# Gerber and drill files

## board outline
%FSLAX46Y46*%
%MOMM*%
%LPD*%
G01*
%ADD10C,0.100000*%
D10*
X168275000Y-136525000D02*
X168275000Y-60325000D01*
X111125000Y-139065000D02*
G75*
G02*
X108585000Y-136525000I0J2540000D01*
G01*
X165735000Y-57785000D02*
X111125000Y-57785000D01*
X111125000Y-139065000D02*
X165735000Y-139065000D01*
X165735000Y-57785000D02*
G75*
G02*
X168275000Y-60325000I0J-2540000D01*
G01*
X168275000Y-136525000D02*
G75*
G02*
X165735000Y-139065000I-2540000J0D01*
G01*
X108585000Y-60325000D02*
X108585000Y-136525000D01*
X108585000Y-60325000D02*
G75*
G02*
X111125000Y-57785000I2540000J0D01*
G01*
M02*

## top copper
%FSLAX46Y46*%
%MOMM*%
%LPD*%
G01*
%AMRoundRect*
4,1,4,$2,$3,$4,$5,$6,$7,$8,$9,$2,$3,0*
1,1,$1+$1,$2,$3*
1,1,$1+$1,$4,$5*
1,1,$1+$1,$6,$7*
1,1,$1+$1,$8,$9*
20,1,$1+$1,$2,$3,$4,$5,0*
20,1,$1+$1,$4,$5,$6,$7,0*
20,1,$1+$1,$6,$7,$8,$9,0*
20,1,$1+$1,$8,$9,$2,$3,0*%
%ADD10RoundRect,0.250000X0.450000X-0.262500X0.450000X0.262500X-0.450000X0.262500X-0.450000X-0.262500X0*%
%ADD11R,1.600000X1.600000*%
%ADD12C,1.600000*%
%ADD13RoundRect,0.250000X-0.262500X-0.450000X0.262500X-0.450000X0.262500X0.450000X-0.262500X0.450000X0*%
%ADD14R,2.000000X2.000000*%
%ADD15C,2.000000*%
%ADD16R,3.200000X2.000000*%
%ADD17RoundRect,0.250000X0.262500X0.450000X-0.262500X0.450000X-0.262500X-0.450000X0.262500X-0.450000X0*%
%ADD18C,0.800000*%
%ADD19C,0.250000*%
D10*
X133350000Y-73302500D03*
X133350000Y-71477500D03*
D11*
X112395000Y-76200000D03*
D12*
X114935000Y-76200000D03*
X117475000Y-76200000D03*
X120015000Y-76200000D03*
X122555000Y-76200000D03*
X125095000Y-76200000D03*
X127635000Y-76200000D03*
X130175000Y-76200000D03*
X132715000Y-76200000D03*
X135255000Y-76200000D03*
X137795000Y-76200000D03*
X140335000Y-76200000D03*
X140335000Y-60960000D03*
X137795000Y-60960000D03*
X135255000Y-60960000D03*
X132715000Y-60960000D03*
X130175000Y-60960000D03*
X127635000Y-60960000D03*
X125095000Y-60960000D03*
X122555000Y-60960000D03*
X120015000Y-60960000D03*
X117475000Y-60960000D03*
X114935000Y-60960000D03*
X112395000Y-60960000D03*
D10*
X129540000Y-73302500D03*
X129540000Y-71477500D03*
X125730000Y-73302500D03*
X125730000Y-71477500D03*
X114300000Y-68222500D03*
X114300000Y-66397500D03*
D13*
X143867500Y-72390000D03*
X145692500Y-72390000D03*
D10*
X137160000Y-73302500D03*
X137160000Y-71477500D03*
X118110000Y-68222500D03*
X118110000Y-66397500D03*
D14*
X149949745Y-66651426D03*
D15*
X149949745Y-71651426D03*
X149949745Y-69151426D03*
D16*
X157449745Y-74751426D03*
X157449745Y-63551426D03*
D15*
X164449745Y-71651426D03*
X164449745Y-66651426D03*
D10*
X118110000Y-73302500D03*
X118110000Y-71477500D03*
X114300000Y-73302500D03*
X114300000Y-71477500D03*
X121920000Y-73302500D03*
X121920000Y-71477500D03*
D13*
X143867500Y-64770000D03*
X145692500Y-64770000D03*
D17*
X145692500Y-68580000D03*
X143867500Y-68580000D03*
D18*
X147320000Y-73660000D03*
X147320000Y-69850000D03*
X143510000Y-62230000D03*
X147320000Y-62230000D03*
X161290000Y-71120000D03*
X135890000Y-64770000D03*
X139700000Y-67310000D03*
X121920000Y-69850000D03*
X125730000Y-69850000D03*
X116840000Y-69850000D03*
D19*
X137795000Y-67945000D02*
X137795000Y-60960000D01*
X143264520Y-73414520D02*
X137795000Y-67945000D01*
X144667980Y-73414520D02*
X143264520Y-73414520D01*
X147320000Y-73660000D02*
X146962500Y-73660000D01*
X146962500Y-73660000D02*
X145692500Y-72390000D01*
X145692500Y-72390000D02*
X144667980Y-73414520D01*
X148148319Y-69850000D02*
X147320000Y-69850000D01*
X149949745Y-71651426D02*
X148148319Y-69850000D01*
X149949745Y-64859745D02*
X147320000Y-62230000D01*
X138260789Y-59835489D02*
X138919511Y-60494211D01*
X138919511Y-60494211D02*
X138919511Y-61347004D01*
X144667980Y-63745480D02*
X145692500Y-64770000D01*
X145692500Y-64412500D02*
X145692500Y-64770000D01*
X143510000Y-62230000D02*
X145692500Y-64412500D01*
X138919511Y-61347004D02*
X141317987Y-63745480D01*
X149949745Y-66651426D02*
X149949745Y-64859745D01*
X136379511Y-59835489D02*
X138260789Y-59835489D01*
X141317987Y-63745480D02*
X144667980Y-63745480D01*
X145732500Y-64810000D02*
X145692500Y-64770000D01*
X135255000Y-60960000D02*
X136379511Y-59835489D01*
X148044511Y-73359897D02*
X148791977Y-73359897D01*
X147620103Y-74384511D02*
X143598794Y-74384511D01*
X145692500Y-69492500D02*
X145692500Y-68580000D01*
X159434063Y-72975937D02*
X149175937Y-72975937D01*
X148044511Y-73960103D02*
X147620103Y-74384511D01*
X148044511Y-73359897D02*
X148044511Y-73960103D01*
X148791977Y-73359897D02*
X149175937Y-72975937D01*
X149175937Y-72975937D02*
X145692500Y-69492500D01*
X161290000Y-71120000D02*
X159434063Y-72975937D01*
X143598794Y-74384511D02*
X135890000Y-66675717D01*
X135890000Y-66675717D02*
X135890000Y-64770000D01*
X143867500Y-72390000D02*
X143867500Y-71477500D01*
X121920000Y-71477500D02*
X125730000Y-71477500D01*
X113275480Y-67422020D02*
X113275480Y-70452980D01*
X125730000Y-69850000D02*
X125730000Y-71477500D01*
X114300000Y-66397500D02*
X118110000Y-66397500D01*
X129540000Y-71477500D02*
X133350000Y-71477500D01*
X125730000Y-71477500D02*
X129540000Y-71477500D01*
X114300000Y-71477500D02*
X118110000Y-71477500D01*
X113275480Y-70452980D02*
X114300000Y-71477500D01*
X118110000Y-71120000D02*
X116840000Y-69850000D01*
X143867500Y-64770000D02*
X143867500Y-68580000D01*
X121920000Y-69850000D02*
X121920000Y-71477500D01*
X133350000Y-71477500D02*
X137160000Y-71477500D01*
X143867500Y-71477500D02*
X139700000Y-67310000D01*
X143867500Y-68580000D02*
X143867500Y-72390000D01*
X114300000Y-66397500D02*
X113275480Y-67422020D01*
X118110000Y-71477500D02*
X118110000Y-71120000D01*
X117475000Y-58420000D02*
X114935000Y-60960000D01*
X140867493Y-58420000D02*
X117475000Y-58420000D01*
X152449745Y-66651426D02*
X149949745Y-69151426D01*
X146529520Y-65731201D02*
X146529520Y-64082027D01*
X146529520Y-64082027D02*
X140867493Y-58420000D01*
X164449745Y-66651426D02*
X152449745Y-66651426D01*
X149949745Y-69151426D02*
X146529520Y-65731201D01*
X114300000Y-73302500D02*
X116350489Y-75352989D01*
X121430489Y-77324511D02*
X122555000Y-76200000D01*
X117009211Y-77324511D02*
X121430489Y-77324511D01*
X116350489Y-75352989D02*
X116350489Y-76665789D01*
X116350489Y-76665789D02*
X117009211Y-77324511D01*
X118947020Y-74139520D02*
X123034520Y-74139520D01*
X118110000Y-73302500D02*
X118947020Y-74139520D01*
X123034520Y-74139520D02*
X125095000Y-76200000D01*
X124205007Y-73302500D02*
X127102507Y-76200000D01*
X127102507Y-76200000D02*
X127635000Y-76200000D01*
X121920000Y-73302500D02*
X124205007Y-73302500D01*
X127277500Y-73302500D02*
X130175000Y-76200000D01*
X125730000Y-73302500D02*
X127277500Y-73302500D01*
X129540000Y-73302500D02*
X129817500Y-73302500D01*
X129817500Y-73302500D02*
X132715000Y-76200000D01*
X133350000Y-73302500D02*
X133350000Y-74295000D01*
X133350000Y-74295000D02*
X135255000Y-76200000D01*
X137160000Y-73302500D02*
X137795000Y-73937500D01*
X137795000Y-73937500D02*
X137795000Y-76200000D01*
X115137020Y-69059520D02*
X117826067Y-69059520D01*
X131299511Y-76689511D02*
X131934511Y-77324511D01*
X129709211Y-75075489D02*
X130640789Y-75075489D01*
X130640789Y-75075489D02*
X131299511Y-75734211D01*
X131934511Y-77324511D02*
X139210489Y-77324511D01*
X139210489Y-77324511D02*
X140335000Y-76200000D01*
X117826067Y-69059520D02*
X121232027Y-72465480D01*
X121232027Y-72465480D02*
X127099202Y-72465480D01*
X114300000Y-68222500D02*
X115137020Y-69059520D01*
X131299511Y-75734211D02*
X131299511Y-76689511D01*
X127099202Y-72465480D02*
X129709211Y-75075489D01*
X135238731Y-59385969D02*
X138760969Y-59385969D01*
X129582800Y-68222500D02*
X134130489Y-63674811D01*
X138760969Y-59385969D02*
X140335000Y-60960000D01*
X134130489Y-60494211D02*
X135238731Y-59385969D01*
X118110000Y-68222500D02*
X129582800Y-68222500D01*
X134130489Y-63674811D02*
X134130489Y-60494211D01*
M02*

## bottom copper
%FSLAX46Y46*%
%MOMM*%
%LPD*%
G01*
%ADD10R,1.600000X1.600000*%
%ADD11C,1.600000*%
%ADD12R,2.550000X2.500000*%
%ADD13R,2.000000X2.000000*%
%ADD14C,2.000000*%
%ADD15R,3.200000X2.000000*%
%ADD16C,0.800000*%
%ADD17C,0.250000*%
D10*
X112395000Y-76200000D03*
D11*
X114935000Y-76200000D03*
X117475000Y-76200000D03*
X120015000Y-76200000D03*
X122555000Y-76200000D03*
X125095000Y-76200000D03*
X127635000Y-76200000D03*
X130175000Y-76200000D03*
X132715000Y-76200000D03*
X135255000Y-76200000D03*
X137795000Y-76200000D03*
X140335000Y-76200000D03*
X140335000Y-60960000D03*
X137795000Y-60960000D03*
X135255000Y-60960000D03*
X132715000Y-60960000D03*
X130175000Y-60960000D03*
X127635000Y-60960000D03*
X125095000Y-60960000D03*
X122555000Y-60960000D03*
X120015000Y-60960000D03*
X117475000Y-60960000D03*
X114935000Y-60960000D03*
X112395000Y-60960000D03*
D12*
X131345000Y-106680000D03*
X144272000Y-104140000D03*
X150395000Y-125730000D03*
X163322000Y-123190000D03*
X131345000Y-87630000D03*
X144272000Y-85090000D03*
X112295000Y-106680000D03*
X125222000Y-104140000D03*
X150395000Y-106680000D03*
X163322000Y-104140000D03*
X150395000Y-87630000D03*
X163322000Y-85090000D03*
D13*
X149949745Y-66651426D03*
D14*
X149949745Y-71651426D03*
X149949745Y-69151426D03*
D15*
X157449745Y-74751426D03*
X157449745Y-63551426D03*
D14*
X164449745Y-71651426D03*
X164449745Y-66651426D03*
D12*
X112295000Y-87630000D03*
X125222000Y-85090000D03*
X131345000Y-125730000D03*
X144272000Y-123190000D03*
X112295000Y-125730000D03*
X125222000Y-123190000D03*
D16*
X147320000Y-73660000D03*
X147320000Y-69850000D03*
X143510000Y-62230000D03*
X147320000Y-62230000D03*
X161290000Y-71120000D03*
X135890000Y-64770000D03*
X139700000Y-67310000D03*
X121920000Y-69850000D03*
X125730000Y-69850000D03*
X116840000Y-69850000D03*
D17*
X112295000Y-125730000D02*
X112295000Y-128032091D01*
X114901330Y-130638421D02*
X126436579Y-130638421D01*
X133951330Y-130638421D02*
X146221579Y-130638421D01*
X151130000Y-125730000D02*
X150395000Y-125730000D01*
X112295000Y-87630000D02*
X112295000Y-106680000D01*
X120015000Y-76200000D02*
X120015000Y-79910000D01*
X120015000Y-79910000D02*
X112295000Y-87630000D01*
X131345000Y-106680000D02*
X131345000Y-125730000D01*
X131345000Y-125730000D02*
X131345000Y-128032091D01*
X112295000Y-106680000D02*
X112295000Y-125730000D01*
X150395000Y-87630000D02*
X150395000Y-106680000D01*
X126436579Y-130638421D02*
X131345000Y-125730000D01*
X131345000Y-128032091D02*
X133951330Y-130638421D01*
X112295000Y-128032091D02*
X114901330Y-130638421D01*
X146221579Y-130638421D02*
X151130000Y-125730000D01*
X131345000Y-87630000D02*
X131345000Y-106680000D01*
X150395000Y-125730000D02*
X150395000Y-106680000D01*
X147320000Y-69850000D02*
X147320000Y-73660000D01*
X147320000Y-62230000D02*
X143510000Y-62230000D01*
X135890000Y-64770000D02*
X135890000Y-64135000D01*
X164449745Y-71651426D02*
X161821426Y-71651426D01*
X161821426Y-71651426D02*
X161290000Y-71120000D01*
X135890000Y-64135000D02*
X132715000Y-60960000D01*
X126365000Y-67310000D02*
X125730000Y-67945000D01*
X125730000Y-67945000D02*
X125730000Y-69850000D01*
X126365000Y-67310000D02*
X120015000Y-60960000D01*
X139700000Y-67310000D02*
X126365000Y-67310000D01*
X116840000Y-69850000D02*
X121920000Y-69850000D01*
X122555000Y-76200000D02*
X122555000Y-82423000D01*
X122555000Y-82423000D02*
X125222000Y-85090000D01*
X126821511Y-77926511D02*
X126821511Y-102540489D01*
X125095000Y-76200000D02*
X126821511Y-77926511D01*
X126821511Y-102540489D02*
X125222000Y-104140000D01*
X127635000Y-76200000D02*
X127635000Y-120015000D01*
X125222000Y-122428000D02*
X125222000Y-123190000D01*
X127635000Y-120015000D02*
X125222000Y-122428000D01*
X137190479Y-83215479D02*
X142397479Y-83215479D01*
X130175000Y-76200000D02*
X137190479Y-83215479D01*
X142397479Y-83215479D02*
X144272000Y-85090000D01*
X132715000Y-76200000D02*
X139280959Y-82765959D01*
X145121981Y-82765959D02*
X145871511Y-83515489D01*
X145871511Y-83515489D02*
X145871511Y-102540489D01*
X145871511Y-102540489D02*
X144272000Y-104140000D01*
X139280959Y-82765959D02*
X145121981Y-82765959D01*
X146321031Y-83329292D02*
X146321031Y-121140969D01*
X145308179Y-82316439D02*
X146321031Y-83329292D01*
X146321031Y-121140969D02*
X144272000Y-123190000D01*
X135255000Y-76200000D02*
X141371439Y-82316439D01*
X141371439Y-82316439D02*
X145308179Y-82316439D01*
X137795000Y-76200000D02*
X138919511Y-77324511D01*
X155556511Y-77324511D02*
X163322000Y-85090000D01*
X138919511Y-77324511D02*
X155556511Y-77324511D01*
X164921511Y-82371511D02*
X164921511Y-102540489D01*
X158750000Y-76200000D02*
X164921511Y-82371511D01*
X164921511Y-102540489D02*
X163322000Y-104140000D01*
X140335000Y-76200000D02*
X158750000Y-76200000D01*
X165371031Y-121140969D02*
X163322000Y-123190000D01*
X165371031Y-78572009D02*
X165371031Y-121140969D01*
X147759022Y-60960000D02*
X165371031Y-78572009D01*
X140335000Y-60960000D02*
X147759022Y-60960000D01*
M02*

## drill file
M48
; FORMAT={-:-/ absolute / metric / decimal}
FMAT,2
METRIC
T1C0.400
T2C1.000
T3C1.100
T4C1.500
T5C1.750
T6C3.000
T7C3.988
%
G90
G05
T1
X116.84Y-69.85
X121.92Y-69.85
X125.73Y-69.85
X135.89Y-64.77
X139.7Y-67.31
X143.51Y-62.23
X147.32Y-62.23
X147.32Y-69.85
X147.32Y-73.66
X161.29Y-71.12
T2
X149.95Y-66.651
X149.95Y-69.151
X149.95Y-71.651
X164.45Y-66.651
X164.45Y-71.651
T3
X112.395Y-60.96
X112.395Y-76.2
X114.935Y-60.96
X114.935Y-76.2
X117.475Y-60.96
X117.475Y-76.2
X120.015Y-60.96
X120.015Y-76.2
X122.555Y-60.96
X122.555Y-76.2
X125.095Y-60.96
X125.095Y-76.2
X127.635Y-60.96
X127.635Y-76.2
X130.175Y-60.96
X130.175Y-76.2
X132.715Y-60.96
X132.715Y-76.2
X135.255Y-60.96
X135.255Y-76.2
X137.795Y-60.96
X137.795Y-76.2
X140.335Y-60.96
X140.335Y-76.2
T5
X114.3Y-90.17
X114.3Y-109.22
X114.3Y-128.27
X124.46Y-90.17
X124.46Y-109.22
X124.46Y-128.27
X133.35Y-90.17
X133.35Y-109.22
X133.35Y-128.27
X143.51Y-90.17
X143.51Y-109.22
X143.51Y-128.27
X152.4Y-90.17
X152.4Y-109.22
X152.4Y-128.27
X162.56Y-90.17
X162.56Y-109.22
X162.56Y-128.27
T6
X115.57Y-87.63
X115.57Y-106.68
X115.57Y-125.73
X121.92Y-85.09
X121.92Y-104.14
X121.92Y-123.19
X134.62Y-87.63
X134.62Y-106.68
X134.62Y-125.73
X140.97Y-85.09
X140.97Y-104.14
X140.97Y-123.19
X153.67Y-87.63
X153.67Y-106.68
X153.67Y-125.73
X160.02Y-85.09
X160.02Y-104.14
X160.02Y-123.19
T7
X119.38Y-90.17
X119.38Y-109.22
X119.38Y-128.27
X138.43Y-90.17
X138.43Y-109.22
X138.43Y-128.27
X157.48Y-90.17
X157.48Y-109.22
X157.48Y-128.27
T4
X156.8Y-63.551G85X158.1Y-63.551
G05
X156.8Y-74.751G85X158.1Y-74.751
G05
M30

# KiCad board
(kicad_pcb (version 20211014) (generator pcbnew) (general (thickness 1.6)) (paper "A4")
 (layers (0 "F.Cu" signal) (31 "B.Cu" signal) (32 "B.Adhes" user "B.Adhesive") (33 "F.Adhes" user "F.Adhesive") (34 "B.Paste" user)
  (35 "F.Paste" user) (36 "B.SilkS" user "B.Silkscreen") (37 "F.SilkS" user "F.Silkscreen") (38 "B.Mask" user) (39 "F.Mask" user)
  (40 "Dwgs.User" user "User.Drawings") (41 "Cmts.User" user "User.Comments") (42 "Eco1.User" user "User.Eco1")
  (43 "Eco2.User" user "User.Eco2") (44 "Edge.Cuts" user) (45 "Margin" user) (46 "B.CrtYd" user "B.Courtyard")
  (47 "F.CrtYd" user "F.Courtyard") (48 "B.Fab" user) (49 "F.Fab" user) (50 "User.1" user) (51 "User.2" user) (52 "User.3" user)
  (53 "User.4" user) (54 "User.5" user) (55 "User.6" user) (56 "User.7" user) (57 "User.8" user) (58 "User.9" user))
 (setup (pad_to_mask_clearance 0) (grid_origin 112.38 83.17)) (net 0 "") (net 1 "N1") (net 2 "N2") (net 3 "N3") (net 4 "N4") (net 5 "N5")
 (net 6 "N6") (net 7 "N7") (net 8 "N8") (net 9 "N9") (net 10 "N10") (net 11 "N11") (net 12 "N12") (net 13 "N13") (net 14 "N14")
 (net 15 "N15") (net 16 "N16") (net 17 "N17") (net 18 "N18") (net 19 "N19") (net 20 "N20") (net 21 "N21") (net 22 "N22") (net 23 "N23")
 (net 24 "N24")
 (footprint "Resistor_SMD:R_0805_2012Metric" (layer "F.Cu") (at 133.35 72.39 90)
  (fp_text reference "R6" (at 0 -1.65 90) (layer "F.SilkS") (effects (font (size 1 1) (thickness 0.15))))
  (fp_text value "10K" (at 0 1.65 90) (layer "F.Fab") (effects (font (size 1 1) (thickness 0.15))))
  (pad "1" smd roundrect locked (at -0.9125 0 90) (size 1.025 1.4) (layers "F.Cu" "F.Paste" "F.Mask") (roundrect_rratio 0.243902439)
   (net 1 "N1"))
  (pad "2" smd roundrect locked (at 0.9125 0 90) (size 1.025 1.4) (layers "F.Cu" "F.Paste" "F.Mask") (roundrect_rratio 0.243902439)
   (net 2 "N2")))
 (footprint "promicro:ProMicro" (layer "F.Cu") (at 126.365 68.58)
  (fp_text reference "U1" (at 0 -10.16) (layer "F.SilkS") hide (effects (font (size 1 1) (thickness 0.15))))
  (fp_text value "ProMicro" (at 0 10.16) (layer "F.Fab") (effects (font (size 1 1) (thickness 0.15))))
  (pad "1" thru_hole rect locked (at -13.97 7.62) (size 1.6 1.6) (drill 1.1) (layers *.Cu *.Mask "F.SilkS") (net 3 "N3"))
  (pad "2" thru_hole circle locked (at -11.43 7.62) (size 1.6 1.6) (drill 1.1) (layers *.Cu *.Mask "F.SilkS") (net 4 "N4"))
  (pad "3" thru_hole circle locked (at -8.89 7.62) (size 1.6 1.6) (drill 1.1) (layers *.Cu *.Mask "F.SilkS") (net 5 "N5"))
  (pad "4" thru_hole circle locked (at -6.35 7.62) (size 1.6 1.6) (drill 1.1) (layers *.Cu *.Mask "F.SilkS") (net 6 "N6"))
  (pad "5" thru_hole circle locked (at -3.81 7.62) (size 1.6 1.6) (drill 1.1) (layers *.Cu *.Mask "F.SilkS") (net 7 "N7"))
  (pad "6" thru_hole circle locked (at -1.27 7.62) (size 1.6 1.6) (drill 1.1) (layers *.Cu *.Mask "F.SilkS") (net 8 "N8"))
  (pad "7" thru_hole circle locked (at 1.27 7.62) (size 1.6 1.6) (drill 1.1) (layers *.Cu *.Mask "F.SilkS") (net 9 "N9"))
  (pad "8" thru_hole circle locked (at 3.81 7.62) (size 1.6 1.6) (drill 1.1) (layers *.Cu *.Mask "F.SilkS") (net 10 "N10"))
  (pad "9" thru_hole circle locked (at 6.35 7.62) (size 1.6 1.6) (drill 1.1) (layers *.Cu *.Mask "F.SilkS") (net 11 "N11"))
  (pad "10" thru_hole circle locked (at 8.89 7.62) (size 1.6 1.6) (drill 1.1) (layers *.Cu *.Mask "F.SilkS") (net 1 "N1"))
  (pad "11" thru_hole circle locked (at 11.43 7.62) (size 1.6 1.6) (drill 1.1) (layers *.Cu *.Mask "F.SilkS") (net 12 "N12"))
  (pad "12" thru_hole circle locked (at 13.97 7.62) (size 1.6 1.6) (drill 1.1) (layers *.Cu *.Mask "F.SilkS") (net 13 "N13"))
  (pad "13" thru_hole circle locked (at 13.97 -7.62) (size 1.6 1.6) (drill 1.1) (layers *.Cu *.Mask "F.SilkS") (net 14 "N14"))
  (pad "14" thru_hole circle locked (at 11.43 -7.62) (size 1.6 1.6) (drill 1.1) (layers *.Cu *.Mask "F.SilkS") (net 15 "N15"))
  (pad "15" thru_hole circle locked (at 8.89 -7.62) (size 1.6 1.6) (drill 1.1) (layers *.Cu *.Mask "F.SilkS") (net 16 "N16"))
  (pad "16" thru_hole circle locked (at 6.35 -7.62) (size 1.6 1.6) (drill 1.1) (layers *.Cu *.Mask "F.SilkS") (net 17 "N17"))
  (pad "17" thru_hole circle locked (at 3.81 -7.62) (size 1.6 1.6) (drill 1.1) (layers *.Cu *.Mask "F.SilkS") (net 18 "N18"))
  (pad "18" thru_hole circle locked (at 1.27 -7.62) (size 1.6 1.6) (drill 1.1) (layers *.Cu *.Mask "F.SilkS") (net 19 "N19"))
  (pad "19" thru_hole circle locked (at -1.27 -7.62) (size 1.6 1.6) (drill 1.1) (layers *.Cu *.Mask "F.SilkS") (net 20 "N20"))
  (pad "20" thru_hole circle locked (at -3.81 -7.62) (size 1.6 1.6) (drill 1.1) (layers *.Cu *.Mask "F.SilkS") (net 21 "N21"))
  (pad "21" thru_hole circle locked (at -6.35 -7.62) (size 1.6 1.6) (drill 1.1) (layers *.Cu *.Mask "F.SilkS") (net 2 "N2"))
  (pad "22" thru_hole circle locked (at -8.89 -7.62) (size 1.6 1.6) (drill 1.1) (layers *.Cu *.Mask "F.SilkS") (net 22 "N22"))
  (pad "23" thru_hole circle locked (at -11.43 -7.62) (size 1.6 1.6) (drill 1.1) (layers *.Cu *.Mask "F.SilkS") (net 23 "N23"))
  (pad "24" thru_hole circle locked (at -13.97 -7.62) (size 1.6 1.6) (drill 1.1) (layers *.Cu *.Mask "F.SilkS") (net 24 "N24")))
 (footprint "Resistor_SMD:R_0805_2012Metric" (layer "F.Cu") (at 129.54 72.39 90)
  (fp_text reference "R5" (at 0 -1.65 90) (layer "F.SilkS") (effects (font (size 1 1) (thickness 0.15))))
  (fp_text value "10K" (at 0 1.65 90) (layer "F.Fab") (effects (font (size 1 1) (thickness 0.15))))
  (pad "1" smd roundrect locked (at -0.9125 0 90) (size 1.025 1.4) (layers "F.Cu" "F.Paste" "F.Mask") (roundrect_rratio 0.243902439)
   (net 11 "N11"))
  (pad "2" smd roundrect locked (at 0.9125 0 90) (size 1.025 1.4) (layers "F.Cu" "F.Paste" "F.Mask") (roundrect_rratio 0.243902439)
   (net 2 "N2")))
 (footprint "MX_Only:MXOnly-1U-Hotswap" (layer "F.Cu") (at 138.43 109.22)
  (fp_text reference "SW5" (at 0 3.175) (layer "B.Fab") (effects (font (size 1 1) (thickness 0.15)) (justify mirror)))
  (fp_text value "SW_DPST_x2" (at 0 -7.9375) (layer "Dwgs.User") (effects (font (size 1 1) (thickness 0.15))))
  (pad "" np_thru_hole circle locked (at -5.08 0 48.0996) (size 1.75 1.75) (drill 1.75) (layers *.Cu *.Mask))
  (pad "" np_thru_hole circle locked (at 0 0) (size 3.9878 3.9878) (drill 3.9878) (layers *.Cu *.Mask))
  (pad "" np_thru_hole circle locked (at -3.81 -2.54) (size 3 3) (drill 3) (layers *.Cu *.Mask))
  (pad "" np_thru_hole circle locked (at 2.54 -5.08) (size 3 3) (drill 3) (layers *.Cu *.Mask))
  (pad "" np_thru_hole circle locked (at 5.08 0 48.0996) (size 1.75 1.75) (drill 1.75) (layers *.Cu *.Mask))
  (pad "1" smd rect locked (at -7.085 -2.54) (size 2.55 2.5) (layers "B.Cu" "B.Paste" "B.Mask") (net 6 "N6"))
  (pad "2" smd rect locked (at 5.842 -5.08) (size 2.55 2.5) (layers "B.Cu" "B.Paste" "B.Mask") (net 11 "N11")))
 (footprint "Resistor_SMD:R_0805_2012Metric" (layer "F.Cu") (at 125.73 72.39 90)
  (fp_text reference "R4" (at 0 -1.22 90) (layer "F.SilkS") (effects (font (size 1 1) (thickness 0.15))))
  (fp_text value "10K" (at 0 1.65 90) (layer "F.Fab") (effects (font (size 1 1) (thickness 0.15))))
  (pad "1" smd roundrect locked (at -0.9125 0 90) (size 1.025 1.4) (layers "F.Cu" "F.Paste" "F.Mask") (roundrect_rratio 0.243902439)
   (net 10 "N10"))
  (pad "2" smd roundrect locked (at 0.9125 0 90) (size 1.025 1.4) (layers "F.Cu" "F.Paste" "F.Mask") (roundrect_rratio 0.243902439)
   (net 2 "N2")))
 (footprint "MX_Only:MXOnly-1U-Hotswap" (layer "F.Cu") (at 157.48 128.27)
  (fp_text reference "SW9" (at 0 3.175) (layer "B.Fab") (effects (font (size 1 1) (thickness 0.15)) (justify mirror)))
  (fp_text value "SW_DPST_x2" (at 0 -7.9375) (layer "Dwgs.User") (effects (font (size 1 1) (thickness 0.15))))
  (pad "" np_thru_hole circle locked (at -5.08 0 48.0996) (size 1.75 1.75) (drill 1.75) (layers *.Cu *.Mask))
  (pad "" np_thru_hole circle locked (at 0 0) (size 3.9878 3.9878) (drill 3.9878) (layers *.Cu *.Mask))
  (pad "" np_thru_hole circle locked (at -3.81 -2.54) (size 3 3) (drill 3) (layers *.Cu *.Mask))
  (pad "" np_thru_hole circle locked (at 5.08 0 48.0996) (size 1.75 1.75) (drill 1.75) (layers *.Cu *.Mask))
  (pad "" np_thru_hole circle locked (at 2.54 -5.08) (size 3 3) (drill 3) (layers *.Cu *.Mask))
  (pad "1" smd rect locked (at -7.085 -2.54) (size 2.55 2.5) (layers "B.Cu" "B.Paste" "B.Mask") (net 6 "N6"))
  (pad "2" smd rect locked (at 5.842 -5.08) (size 2.55 2.5) (layers "B.Cu" "B.Paste" "B.Mask") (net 14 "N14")))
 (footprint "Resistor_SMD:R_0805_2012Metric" (layer "F.Cu") (at 114.3 67.31 90)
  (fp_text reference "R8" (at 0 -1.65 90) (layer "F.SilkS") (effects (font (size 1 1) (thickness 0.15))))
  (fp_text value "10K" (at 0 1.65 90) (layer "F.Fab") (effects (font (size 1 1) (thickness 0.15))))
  (pad "1" smd roundrect locked (at -0.9125 0 90) (size 1.025 1.4) (layers "F.Cu" "F.Paste" "F.Mask") (roundrect_rratio 0.243902439)
   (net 13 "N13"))
  (pad "2" smd roundrect locked (at 0.9125 0 90) (size 1.025 1.4) (layers "F.Cu" "F.Paste" "F.Mask") (roundrect_rratio 0.243902439)
   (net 2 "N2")))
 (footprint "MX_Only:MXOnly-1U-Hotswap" (layer "F.Cu") (at 138.43 90.17)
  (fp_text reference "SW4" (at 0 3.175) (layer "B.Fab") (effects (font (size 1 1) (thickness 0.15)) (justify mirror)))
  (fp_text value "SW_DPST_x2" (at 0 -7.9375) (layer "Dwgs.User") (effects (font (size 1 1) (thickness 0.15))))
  (pad "" np_thru_hole circle locked (at -3.81 -2.54) (size 3 3) (drill 3) (layers *.Cu *.Mask))
  (pad "" np_thru_hole circle locked (at 5.08 0 48.0996) (size 1.75 1.75) (drill 1.75) (layers *.Cu *.Mask))
  (pad "" np_thru_hole circle locked (at 0 0) (size 3.9878 3.9878) (drill 3.9878) (layers *.Cu *.Mask))
  (pad "" np_thru_hole circle locked (at 2.54 -5.08) (size 3 3) (drill 3) (layers *.Cu *.Mask))
  (pad "" np_thru_hole circle locked (at -5.08 0 48.0996) (size 1.75 1.75) (drill 1.75) (layers *.Cu *.Mask))
  (pad "1" smd rect locked (at -7.085 -2.54) (size 2.55 2.5) (layers "B.Cu" "B.Paste" "B.Mask") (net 6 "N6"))
  (pad "2" smd rect locked (at 5.842 -5.08) (size 2.55 2.5) (layers "B.Cu" "B.Paste" "B.Mask") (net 10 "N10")))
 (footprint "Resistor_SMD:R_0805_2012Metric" (layer "F.Cu") (at 144.78 72.39)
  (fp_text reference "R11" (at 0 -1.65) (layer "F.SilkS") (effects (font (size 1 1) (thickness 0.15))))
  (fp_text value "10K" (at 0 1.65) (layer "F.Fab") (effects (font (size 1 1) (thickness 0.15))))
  (pad "1" smd roundrect locked (at -0.9125 0) (size 1.025 1.4) (layers "F.Cu" "F.Paste" "F.Mask") (roundrect_rratio 0.243902439)
   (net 2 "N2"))
  (pad "2" smd roundrect locked (at 0.9125 0) (size 1.025 1.4) (layers "F.Cu" "F.Paste" "F.Mask") (roundrect_rratio 0.243902439)
   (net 15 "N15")))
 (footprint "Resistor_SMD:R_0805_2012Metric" (layer "F.Cu") (at 137.16 72.39 90)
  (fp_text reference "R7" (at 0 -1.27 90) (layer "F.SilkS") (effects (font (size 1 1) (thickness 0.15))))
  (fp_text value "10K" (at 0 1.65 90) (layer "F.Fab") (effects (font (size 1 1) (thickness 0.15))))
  (pad "1" smd roundrect locked (at -0.9125 0 90) (size 1.025 1.4) (layers "F.Cu" "F.Paste" "F.Mask") (roundrect_rratio 0.243902439)
   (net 12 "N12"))
  (pad "2" smd roundrect locked (at 0.9125 0 90) (size 1.025 1.4) (layers "F.Cu" "F.Paste" "F.Mask") (roundrect_rratio 0.243902439)
   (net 2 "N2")))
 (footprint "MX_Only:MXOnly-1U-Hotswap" (layer "F.Cu") (at 119.38 109.22)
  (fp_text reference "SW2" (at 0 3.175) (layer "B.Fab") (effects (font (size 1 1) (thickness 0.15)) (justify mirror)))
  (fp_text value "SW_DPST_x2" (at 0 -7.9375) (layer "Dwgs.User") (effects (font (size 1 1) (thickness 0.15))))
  (pad "" np_thru_hole circle locked (at 2.54 -5.08) (size 3 3) (drill 3) (layers *.Cu *.Mask))
  (pad "" np_thru_hole circle locked (at 5.08 0 48.0996) (size 1.75 1.75) (drill 1.75) (layers *.Cu *.Mask))
  (pad "" np_thru_hole circle locked (at 0 0) (size 3.9878 3.9878) (drill 3.9878) (layers *.Cu *.Mask))
  (pad "" np_thru_hole circle locked (at -3.81 -2.54) (size 3 3) (drill 3) (layers *.Cu *.Mask))
  (pad "" np_thru_hole circle locked (at -5.08 0 48.0996) (size 1.75 1.75) (drill 1.75) (layers *.Cu *.Mask))
  (pad "1" smd rect locked (at -7.085 -2.54) (size 2.55 2.5) (layers "B.Cu" "B.Paste" "B.Mask") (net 6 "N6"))
  (pad "2" smd rect locked (at 5.842 -5.08) (size 2.55 2.5) (layers "B.Cu" "B.Paste" "B.Mask") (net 8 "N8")))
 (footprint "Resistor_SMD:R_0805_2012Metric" (layer "F.Cu") (at 118.11 67.31 90)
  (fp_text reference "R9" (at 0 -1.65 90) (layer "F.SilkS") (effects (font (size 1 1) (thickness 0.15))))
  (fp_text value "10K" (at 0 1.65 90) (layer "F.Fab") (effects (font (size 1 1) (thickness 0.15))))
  (pad "1" smd roundrect locked (at -0.9125 0 90) (size 1.025 1.4) (layers "F.Cu" "F.Paste" "F.Mask") (roundrect_rratio 0.243902439)
   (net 14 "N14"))
  (pad "2" smd roundrect locked (at 0.9125 0 90) (size 1.025 1.4) (layers "F.Cu" "F.Paste" "F.Mask") (roundrect_rratio 0.243902439)
   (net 2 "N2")))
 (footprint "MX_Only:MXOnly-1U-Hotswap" (layer "F.Cu") (at 157.48 109.22)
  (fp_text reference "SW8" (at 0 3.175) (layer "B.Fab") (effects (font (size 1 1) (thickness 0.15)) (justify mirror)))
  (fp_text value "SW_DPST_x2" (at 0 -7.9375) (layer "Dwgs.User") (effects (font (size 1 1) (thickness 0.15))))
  (pad "" np_thru_hole circle locked (at 2.54 -5.08) (size 3 3) (drill 3) (layers *.Cu *.Mask))
  (pad "" np_thru_hole circle locked (at 5.08 0 48.0996) (size 1.75 1.75) (drill 1.75) (layers *.Cu *.Mask))
  (pad "" np_thru_hole circle locked (at -5.08 0 48.0996) (size 1.75 1.75) (drill 1.75) (layers *.Cu *.Mask))
  (pad "" np_thru_hole circle locked (at -3.81 -2.54) (size 3 3) (drill 3) (layers *.Cu *.Mask))
  (pad "" np_thru_hole circle locked (at 0 0) (size 3.9878 3.9878) (drill 3.9878) (layers *.Cu *.Mask))
  (pad "1" smd rect locked (at -7.085 -2.54) (size 2.55 2.5) (layers "B.Cu" "B.Paste" "B.Mask") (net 6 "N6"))
  (pad "2" smd rect locked (at 5.842 -5.08) (size 2.55 2.5) (layers "B.Cu" "B.Paste" "B.Mask") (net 13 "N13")))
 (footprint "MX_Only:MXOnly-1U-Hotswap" (layer "F.Cu") (at 157.48 90.17)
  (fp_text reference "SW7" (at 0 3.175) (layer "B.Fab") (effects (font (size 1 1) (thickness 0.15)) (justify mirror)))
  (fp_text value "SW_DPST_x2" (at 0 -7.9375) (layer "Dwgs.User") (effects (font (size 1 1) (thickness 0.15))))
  (pad "" np_thru_hole circle locked (at 5.08 0 48.0996) (size 1.75 1.75) (drill 1.75) (layers *.Cu *.Mask))
  (pad "" np_thru_hole circle locked (at -3.81 -2.54) (size 3 3) (drill 3) (layers *.Cu *.Mask))
  (pad "" np_thru_hole circle locked (at 2.54 -5.08) (size 3 3) (drill 3) (layers *.Cu *.Mask))
  (pad "" np_thru_hole circle locked (at -5.08 0 48.0996) (size 1.75 1.75) (drill 1.75) (layers *.Cu *.Mask))
  (pad "" np_thru_hole circle locked (at 0 0) (size 3.9878 3.9878) (drill 3.9878) (layers *.Cu *.Mask))
  (pad "1" smd rect locked (at -7.085 -2.54) (size 2.55 2.5) (layers "B.Cu" "B.Paste" "B.Mask") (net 6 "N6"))
  (pad "2" smd rect locked (at 5.842 -5.08) (size 2.55 2.5) (layers "B.Cu" "B.Paste" "B.Mask") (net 12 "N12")))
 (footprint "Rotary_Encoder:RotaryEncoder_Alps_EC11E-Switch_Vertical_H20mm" (layer "F.Cu") (at 149.949745 66.651426)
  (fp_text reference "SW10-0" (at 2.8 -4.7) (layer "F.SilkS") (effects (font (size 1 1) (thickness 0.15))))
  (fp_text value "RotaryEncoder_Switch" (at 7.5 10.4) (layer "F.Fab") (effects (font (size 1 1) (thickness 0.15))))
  (pad "A" thru_hole rect locked (at 0 0) (size 2 2) (drill 1) (layers *.Cu *.Mask) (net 16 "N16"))
  (pad "B" thru_hole circle locked (at 0 5) (size 2 2) (drill 1) (layers *.Cu *.Mask) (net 15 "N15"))
  (pad "C" thru_hole circle locked (at 0 2.5) (size 2 2) (drill 1) (layers *.Cu *.Mask) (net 23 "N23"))
  (pad "MP" thru_hole rect locked (at 7.5 8.1) (size 3.2 2) (drill oval 2.8 1.5) (layers *.Cu *.Mask))
  (pad "MP" thru_hole rect locked (at 7.5 -3.1) (size 3.2 2) (drill oval 2.8 1.5) (layers *.Cu *.Mask))
  (pad "S1" thru_hole circle locked (at 14.5 5) (size 2 2) (drill 1) (layers *.Cu *.Mask) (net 17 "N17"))
  (pad "S2" thru_hole circle locked (at 14.5 0) (size 2 2) (drill 1) (layers *.Cu *.Mask) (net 23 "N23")))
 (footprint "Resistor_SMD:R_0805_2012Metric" (layer "F.Cu") (at 118.11 72.39 90)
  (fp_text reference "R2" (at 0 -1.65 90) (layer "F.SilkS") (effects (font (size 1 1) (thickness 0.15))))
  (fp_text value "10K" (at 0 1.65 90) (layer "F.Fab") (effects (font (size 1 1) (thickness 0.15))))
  (pad "1" smd roundrect locked (at -0.9125 0 90) (size 1.025 1.4) (layers "F.Cu" "F.Paste" "F.Mask") (roundrect_rratio 0.243902439)
   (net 8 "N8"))
  (pad "2" smd roundrect locked (at 0.9125 0 90) (size 1.025 1.4) (layers "F.Cu" "F.Paste" "F.Mask") (roundrect_rratio 0.243902439)
   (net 2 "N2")))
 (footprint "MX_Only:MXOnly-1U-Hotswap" (layer "F.Cu") (at 119.38 90.17)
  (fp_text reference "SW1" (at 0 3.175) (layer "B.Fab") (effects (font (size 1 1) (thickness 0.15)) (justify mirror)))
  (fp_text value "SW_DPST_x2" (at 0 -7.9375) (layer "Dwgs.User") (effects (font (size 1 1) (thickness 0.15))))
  (pad "" np_thru_hole circle locked (at 5.08 0 48.0996) (size 1.75 1.75) (drill 1.75) (layers *.Cu *.Mask))
  (pad "" np_thru_hole circle locked (at 0 0) (size 3.9878 3.9878) (drill 3.9878) (layers *.Cu *.Mask))
  (pad "" np_thru_hole circle locked (at 2.54 -5.08) (size 3 3) (drill 3) (layers *.Cu *.Mask))
  (pad "" np_thru_hole circle locked (at -3.81 -2.54) (size 3 3) (drill 3) (layers *.Cu *.Mask))
  (pad "" np_thru_hole circle locked (at -5.08 0 48.0996) (size 1.75 1.75) (drill 1.75) (layers *.Cu *.Mask))
  (pad "1" smd rect locked (at -7.085 -2.54) (size 2.55 2.5) (layers "B.Cu" "B.Paste" "B.Mask") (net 6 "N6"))
  (pad "2" smd rect locked (at 5.842 -5.08) (size 2.55 2.5) (layers "B.Cu" "B.Paste" "B.Mask") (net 7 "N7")))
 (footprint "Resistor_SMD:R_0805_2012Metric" (layer "F.Cu") (at 114.3 72.39 90)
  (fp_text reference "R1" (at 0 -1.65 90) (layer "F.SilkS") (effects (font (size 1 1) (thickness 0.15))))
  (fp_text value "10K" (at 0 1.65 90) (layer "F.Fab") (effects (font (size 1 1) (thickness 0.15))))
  (pad "1" smd roundrect locked (at -0.9125 0 90) (size 1.025 1.4) (layers "F.Cu" "F.Paste" "F.Mask") (roundrect_rratio 0.243902439)
   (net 7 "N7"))
  (pad "2" smd roundrect locked (at 0.9125 0 90) (size 1.025 1.4) (layers "F.Cu" "F.Paste" "F.Mask") (roundrect_rratio 0.243902439)
   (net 2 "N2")))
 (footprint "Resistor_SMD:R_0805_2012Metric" (layer "F.Cu") (at 121.92 72.39 90)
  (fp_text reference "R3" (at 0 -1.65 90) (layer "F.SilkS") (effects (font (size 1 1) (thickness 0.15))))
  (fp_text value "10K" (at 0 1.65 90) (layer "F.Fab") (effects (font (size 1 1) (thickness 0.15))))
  (pad "1" smd roundrect locked (at -0.9125 0 90) (size 1.025 1.4) (layers "F.Cu" "F.Paste" "F.Mask") (roundrect_rratio 0.243902439)
   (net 9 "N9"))
  (pad "2" smd roundrect locked (at 0.9125 0 90) (size 1.025 1.4) (layers "F.Cu" "F.Paste" "F.Mask") (roundrect_rratio 0.243902439)
   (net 2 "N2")))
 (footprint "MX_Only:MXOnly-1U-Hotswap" (layer "F.Cu") (at 138.43 128.27)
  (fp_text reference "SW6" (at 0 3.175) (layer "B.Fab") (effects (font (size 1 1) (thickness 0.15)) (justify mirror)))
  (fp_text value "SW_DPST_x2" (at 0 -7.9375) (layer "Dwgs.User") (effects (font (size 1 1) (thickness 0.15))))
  (pad "" np_thru_hole circle locked (at 0 0) (size 3.9878 3.9878) (drill 3.9878) (layers *.Cu *.Mask))
  (pad "" np_thru_hole circle locked (at -5.08 0 48.0996) (size 1.75 1.75) (drill 1.75) (layers *.Cu *.Mask))
  (pad "" np_thru_hole circle locked (at 2.54 -5.08) (size 3 3) (drill 3) (layers *.Cu *.Mask))
  (pad "" np_thru_hole circle locked (at -3.81 -2.54) (size 3 3) (drill 3) (layers *.Cu *.Mask))
  (pad "" np_thru_hole circle locked (at 5.08 0 48.0996) (size 1.75 1.75) (drill 1.75) (layers *.Cu *.Mask))
  (pad "1" smd rect locked (at -7.085 -2.54) (size 2.55 2.5) (layers "B.Cu" "B.Paste" "B.Mask") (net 6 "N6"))
  (pad "2" smd rect locked (at 5.842 -5.08) (size 2.55 2.5) (layers "B.Cu" "B.Paste" "B.Mask") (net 1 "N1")))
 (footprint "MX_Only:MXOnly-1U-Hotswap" (layer "F.Cu") (at 119.38 128.27)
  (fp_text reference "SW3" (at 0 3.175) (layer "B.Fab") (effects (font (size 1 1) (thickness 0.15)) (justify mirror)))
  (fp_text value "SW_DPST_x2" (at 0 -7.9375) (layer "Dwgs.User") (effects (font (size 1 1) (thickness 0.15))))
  (pad "" np_thru_hole circle locked (at 2.54 -5.08) (size 3 3) (drill 3) (layers *.Cu *.Mask))
  (pad "" np_thru_hole circle locked (at -5.08 0 48.0996) (size 1.75 1.75) (drill 1.75) (layers *.Cu *.Mask))
  (pad "" np_thru_hole circle locked (at 0 0) (size 3.9878 3.9878) (drill 3.9878) (layers *.Cu *.Mask))
  (pad "" np_thru_hole circle locked (at 5.08 0 48.0996) (size 1.75 1.75) (drill 1.75) (layers *.Cu *.Mask))
  (pad "" np_thru_hole circle locked (at -3.81 -2.54) (size 3 3) (drill 3) (layers *.Cu *.Mask))
  (pad "1" smd rect locked (at -7.085 -2.54) (size 2.55 2.5) (layers "B.Cu" "B.Paste" "B.Mask") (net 6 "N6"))
  (pad "2" smd rect locked (at 5.842 -5.08) (size 2.55 2.5) (layers "B.Cu" "B.Paste" "B.Mask") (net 9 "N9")))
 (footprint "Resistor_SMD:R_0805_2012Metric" (layer "F.Cu") (at 144.78 64.77)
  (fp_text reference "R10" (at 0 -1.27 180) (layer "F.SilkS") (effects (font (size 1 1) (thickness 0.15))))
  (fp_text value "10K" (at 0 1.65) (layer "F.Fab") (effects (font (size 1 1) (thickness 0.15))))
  (pad "1" smd roundrect locked (at -0.9125 0) (size 1.025 1.4) (layers "F.Cu" "F.Paste" "F.Mask") (roundrect_rratio 0.243902439)
   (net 2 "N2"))
  (pad "2" smd roundrect locked (at 0.9125 0) (size 1.025 1.4) (layers "F.Cu" "F.Paste" "F.Mask") (roundrect_rratio 0.243902439)
   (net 16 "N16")))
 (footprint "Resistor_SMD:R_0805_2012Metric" (layer "F.Cu") (at 144.78 68.58 180)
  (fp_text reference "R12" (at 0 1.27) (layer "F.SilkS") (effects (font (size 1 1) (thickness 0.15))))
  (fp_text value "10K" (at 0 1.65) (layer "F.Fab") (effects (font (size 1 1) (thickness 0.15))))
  (pad "1" smd roundrect locked (at -0.9125 0 180) (size 1.025 1.4) (layers "F.Cu" "F.Paste" "F.Mask") (roundrect_rratio 0.243902439)
   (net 17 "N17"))
  (pad "2" smd roundrect locked (at 0.9125 0 180) (size 1.025 1.4) (layers "F.Cu" "F.Paste" "F.Mask") (roundrect_rratio 0.243902439)
   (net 2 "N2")))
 (gr_line (start 168.275 136.525) (end 168.275 60.325) (layer "Edge.Cuts") (width 0.1))
 (gr_arc (start 111.125 139.065) (mid 109.328949 138.321051) (end 108.585 136.525) (layer "Edge.Cuts") (width 0.1))
 (gr_line (start 165.735 57.785) (end 111.125 57.785) (layer "Edge.Cuts") (width 0.1))
 (gr_line (start 111.125 139.065) (end 165.735 139.065) (layer "Edge.Cuts") (width 0.1))
 (gr_arc (start 165.735 57.785) (mid 167.531051 58.528949) (end 168.275 60.325) (layer "Edge.Cuts") (width 0.1))
 (gr_arc (start 168.275 136.525) (mid 167.531051 138.321051) (end 165.735 139.065) (layer "Edge.Cuts") (width 0.1))
 (gr_line (start 108.585 60.325) (end 108.585 136.525) (layer "Edge.Cuts") (width 0.1))
 (gr_arc (start 108.585 60.325) (mid 109.328949 58.528949) (end 111.125 57.785) (layer "Edge.Cuts") (width 0.1))
 (segment (start 112.295 125.73) (end 112.295 128.032091) (width 0.25) (layer "B.Cu") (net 6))
 (segment (start 114.90133 130.638421) (end 126.436579 130.638421) (width 0.25) (layer "B.Cu") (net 6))
 (segment (start 133.95133 130.638421) (end 146.221579 130.638421) (width 0.25) (layer "B.Cu") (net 6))
 (segment (start 151.13 125.73) (end 150.395 125.73) (width 0.25) (layer "B.Cu") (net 6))
 (segment (start 112.295 87.63) (end 112.295 106.68) (width 0.25) (layer "B.Cu") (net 6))
 (segment (start 120.015 76.2) (end 120.015 79.91) (width 0.25) (layer "B.Cu") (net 6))
 (segment (start 120.015 79.91) (end 112.295 87.63) (width 0.25) (layer "B.Cu") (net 6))
 (segment (start 131.345 106.68) (end 131.345 125.73) (width 0.25) (layer "B.Cu") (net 6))
 (segment (start 131.345 125.73) (end 131.345 128.032091) (width 0.25) (layer "B.Cu") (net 6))
 (segment (start 112.295 106.68) (end 112.295 125.73) (width 0.25) (layer "B.Cu") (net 6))
 (segment (start 150.395 87.63) (end 150.395 106.68) (width 0.25) (layer "B.Cu") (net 6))
 (segment (start 126.436579 130.638421) (end 131.345 125.73) (width 0.25) (layer "B.Cu") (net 6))
 (segment (start 131.345 128.032091) (end 133.95133 130.638421) (width 0.25) (layer "B.Cu") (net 6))
 (segment (start 112.295 128.032091) (end 114.90133 130.638421) (width 0.25) (layer "B.Cu") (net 6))
 (segment (start 146.221579 130.638421) (end 151.13 125.73) (width 0.25) (layer "B.Cu") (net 6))
 (segment (start 131.345 87.63) (end 131.345 106.68) (width 0.25) (layer "B.Cu") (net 6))
 (segment (start 150.395 125.73) (end 150.395 106.68) (width 0.25) (layer "B.Cu") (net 6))
 (segment (start 137.795 67.945) (end 137.795 60.96) (width 0.25) (layer "F.Cu") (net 15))
 (segment (start 143.26452 73.41452) (end 137.795 67.945) (width 0.25) (layer "F.Cu") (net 15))
 (segment (start 144.66798 73.41452) (end 143.26452 73.41452) (width 0.25) (layer "F.Cu") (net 15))
 (segment (start 147.32 73.66) (end 146.9625 73.66) (width 0.25) (layer "F.Cu") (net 15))
 (segment (start 146.9625 73.66) (end 145.6925 72.39) (width 0.25) (layer "F.Cu") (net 15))
 (segment (start 145.6925 72.39) (end 144.66798 73.41452) (width 0.25) (layer "F.Cu") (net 15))
 (segment (start 148.148319 69.85) (end 147.32 69.85) (width 0.25) (layer "F.Cu") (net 15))
 (segment (start 149.949745 71.651426) (end 148.148319 69.85) (width 0.25) (layer "F.Cu") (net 15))
 (via (at 147.32 73.66) (size 0.8) (drill 0.4) (layers "F.Cu" "B.Cu") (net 15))
 (via (at 147.32 69.85) (size 0.8) (drill 0.4) (layers "F.Cu" "B.Cu") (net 15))
 (segment (start 147.32 69.85) (end 147.32 73.66) (width 0.25) (layer "B.Cu") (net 15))
 (segment (start 149.949745 64.859745) (end 147.32 62.23) (width 0.25) (layer "F.Cu") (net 16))
 (segment (start 138.260789 59.835489) (end 138.919511 60.494211) (width 0.25) (layer "F.Cu") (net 16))
 (segment (start 138.919511 60.494211) (end 138.919511 61.347004) (width 0.25) (layer "F.Cu") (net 16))
 (segment (start 144.66798 63.74548) (end 145.6925 64.77) (width 0.25) (layer "F.Cu") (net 16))
 (segment (start 145.6925 64.4125) (end 145.6925 64.77) (width 0.25) (layer "F.Cu") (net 16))
 (segment (start 143.51 62.23) (end 145.6925 64.4125) (width 0.25) (layer "F.Cu") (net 16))
 (segment (start 138.919511 61.347004) (end 141.317987 63.74548) (width 0.25) (layer "F.Cu") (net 16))
 (segment (start 149.949745 66.651426) (end 149.949745 64.859745) (width 0.25) (layer "F.Cu") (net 16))
 (segment (start 136.379511 59.835489) (end 138.260789 59.835489) (width 0.25) (layer "F.Cu") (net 16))
 (segment (start 141.317987 63.74548) (end 144.66798 63.74548) (width 0.25) (layer "F.Cu") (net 16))
 (segment (start 145.7325 64.81) (end 145.6925 64.77) (width 0.25) (layer "F.Cu") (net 16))
 (segment (start 135.255 60.96) (end 136.379511 59.835489) (width 0.25) (layer "F.Cu") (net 16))
 (via (at 143.51 62.23) (size 0.8) (drill 0.4) (layers "F.Cu" "B.Cu") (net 16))
 (via (at 147.32 62.23) (size 0.8) (drill 0.4) (layers "F.Cu" "B.Cu") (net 16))
 (segment (start 147.32 62.23) (end 143.51 62.23) (width 0.25) (layer "B.Cu") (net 16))
 (segment (start 148.044511 73.359897) (end 148.791977 73.359897) (width 0.25) (layer "F.Cu") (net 17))
 (segment (start 147.620103 74.384511) (end 143.598794 74.384511) (width 0.25) (layer "F.Cu") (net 17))
 (segment (start 145.6925 69.4925) (end 145.6925 68.58) (width 0.25) (layer "F.Cu") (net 17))
 (segment (start 159.434063 72.975937) (end 149.175937 72.975937) (width 0.25) (layer "F.Cu") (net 17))
 (segment (start 148.044511 73.960103) (end 147.620103 74.384511) (width 0.25) (layer "F.Cu") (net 17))
 (segment (start 148.044511 73.359897) (end 148.044511 73.960103) (width 0.25) (layer "F.Cu") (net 17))
 (segment (start 148.791977 73.359897) (end 149.175937 72.975937) (width 0.25) (layer "F.Cu") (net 17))
 (segment (start 149.175937 72.975937) (end 145.6925 69.4925) (width 0.25) (layer "F.Cu") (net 17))
 (segment (start 161.29 71.12) (end 159.434063 72.975937) (width 0.25) (layer "F.Cu") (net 17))
 (segment (start 143.598794 74.384511) (end 135.89 66.675717) (width 0.25) (layer "F.Cu") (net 17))
 (segment (start 135.89 66.675717) (end 135.89 64.77) (width 0.25) (layer "F.Cu") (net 17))
 (via (at 161.29 71.12) (size 0.8) (drill 0.4) (layers "F.Cu" "B.Cu") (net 17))
 (via (at 135.89 64.77) (size 0.8) (drill 0.4) (layers "F.Cu" "B.Cu") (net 17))
 (segment (start 135.89 64.77) (end 135.89 64.135) (width 0.25) (layer "B.Cu") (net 17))
 (segment (start 164.449745 71.651426) (end 161.821426 71.651426) (width 0.25) (layer "B.Cu") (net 17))
 (segment (start 161.821426 71.651426) (end 161.29 71.12) (width 0.25) (layer "B.Cu") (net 17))
 (segment (start 135.89 64.135) (end 132.715 60.96) (width 0.25) (layer "B.Cu") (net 17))
 (segment (start 143.8675 72.39) (end 143.8675 71.4775) (width 0.25) (layer "F.Cu") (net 2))
 (segment (start 121.92 71.4775) (end 125.73 71.4775) (width 0.25) (layer "F.Cu") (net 2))
 (segment (start 113.27548 67.42202) (end 113.27548 70.45298) (width 0.25) (layer "F.Cu") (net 2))
 (segment (start 125.73 69.85) (end 125.73 71.4775) (width 0.25) (layer "F.Cu") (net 2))
 (segment (start 114.3 66.3975) (end 118.11 66.3975) (width 0.25) (layer "F.Cu") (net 2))
 (segment (start 129.54 71.4775) (end 133.35 71.4775) (width 0.25) (layer "F.Cu") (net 2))
 (segment (start 125.73 71.4775) (end 129.54 71.4775) (width 0.25) (layer "F.Cu") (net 2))
 (segment (start 114.3 71.4775) (end 118.11 71.4775) (width 0.25) (layer "F.Cu") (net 2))
 (segment (start 113.27548 70.45298) (end 114.3 71.4775) (width 0.25) (layer "F.Cu") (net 2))
 (segment (start 118.11 71.12) (end 116.84 69.85) (width 0.25) (layer "F.Cu") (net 2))
 (segment (start 143.8675 64.77) (end 143.8675 68.58) (width 0.25) (layer "F.Cu") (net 2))
 (segment (start 121.92 69.85) (end 121.92 71.4775) (width 0.25) (layer "F.Cu") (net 2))
 (segment (start 133.35 71.4775) (end 137.16 71.4775) (width 0.25) (layer "F.Cu") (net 2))
 (segment (start 143.8675 71.4775) (end 139.7 67.31) (width 0.25) (layer "F.Cu") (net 2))
 (segment (start 143.8675 68.58) (end 143.8675 72.39) (width 0.25) (layer "F.Cu") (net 2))
 (segment (start 114.3 66.3975) (end 113.27548 67.42202) (width 0.25) (layer "F.Cu") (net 2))
 (segment (start 118.11 71.4775) (end 118.11 71.12) (width 0.25) (layer "F.Cu") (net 2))
 (via (at 139.7 67.31) (size 0.8) (drill 0.4) (layers "F.Cu" "B.Cu") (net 2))
 (via (at 121.92 69.85) (size 0.8) (drill 0.4) (layers "F.Cu" "B.Cu") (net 2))
 (via (at 125.73 69.85) (size 0.8) (drill 0.4) (layers "F.Cu" "B.Cu") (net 2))
 (via (at 116.84 69.85) (size 0.8) (drill 0.4) (layers "F.Cu" "B.Cu") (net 2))
 (segment (start 126.365 67.31) (end 125.73 67.945) (width 0.25) (layer "B.Cu") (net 2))
 (segment (start 125.73 67.945) (end 125.73 69.85) (width 0.25) (layer "B.Cu") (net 2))
 (segment (start 126.365 67.31) (end 120.015 60.96) (width 0.25) (layer "B.Cu") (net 2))
 (segment (start 139.7 67.31) (end 126.365 67.31) (width 0.25) (layer "B.Cu") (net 2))
 (segment (start 116.84 69.85) (end 121.92 69.85) (width 0.25) (layer "B.Cu") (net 2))
 (segment (start 117.475 58.42) (end 114.935 60.96) (width 0.25) (layer "F.Cu") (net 23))
 (segment (start 140.867493 58.42) (end 117.475 58.42) (width 0.25) (layer "F.Cu") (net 23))
 (segment (start 152.449745 66.651426) (end 149.949745 69.151426) (width 0.25) (layer "F.Cu") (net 23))
 (segment (start 146.52952 65.731201) (end 146.52952 64.082027) (width 0.25) (layer "F.Cu") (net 23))
 (segment (start 146.52952 64.082027) (end 140.867493 58.42) (width 0.25) (layer "F.Cu") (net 23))
 (segment (start 164.449745 66.651426) (end 152.449745 66.651426) (width 0.25) (layer "F.Cu") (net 23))
 (segment (start 149.949745 69.151426) (end 146.52952 65.731201) (width 0.25) (layer "F.Cu") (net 23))
 (segment (start 114.3 73.3025) (end 116.350489 75.352989) (width 0.25) (layer "F.Cu") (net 7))
 (segment (start 121.430489 77.324511) (end 122.555 76.2) (width 0.25) (layer "F.Cu") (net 7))
 (segment (start 117.009211 77.324511) (end 121.430489 77.324511) (width 0.25) (layer "F.Cu") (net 7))
 (segment (start 116.350489 75.352989) (end 116.350489 76.665789) (width 0.25) (layer "F.Cu") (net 7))
 (segment (start 116.350489 76.665789) (end 117.009211 77.324511) (width 0.25) (layer "F.Cu") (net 7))
 (segment (start 122.555 76.2) (end 122.555 82.423) (width 0.25) (layer "B.Cu") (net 7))
 (segment (start 122.555 82.423) (end 125.222 85.09) (width 0.25) (layer "B.Cu") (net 7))
 (segment (start 118.94702 74.13952) (end 123.03452 74.13952) (width 0.25) (layer "F.Cu") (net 8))
 (segment (start 118.11 73.3025) (end 118.94702 74.13952) (width 0.25) (layer "F.Cu") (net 8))
 (segment (start 123.03452 74.13952) (end 125.095 76.2) (width 0.25) (layer "F.Cu") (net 8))
 (segment (start 126.821511 77.926511) (end 126.821511 102.540489) (width 0.25) (layer "B.Cu") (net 8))
 (segment (start 125.095 76.2) (end 126.821511 77.926511) (width 0.25) (layer "B.Cu") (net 8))
 (segment (start 126.821511 102.540489) (end 125.222 104.14) (width 0.25) (layer "B.Cu") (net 8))
 (segment (start 124.205007 73.3025) (end 127.102507 76.2) (width 0.25) (layer "F.Cu") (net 9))
 (segment (start 127.102507 76.2) (end 127.635 76.2) (width 0.25) (layer "F.Cu") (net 9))
 (segment (start 121.92 73.3025) (end 124.205007 73.3025) (width 0.25) (layer "F.Cu") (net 9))
 (segment (start 127.635 76.2) (end 127.635 120.015) (width 0.25) (layer "B.Cu") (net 9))
 (segment (start 125.222 122.428) (end 125.222 123.19) (width 0.25) (layer "B.Cu") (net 9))
 (segment (start 127.635 120.015) (end 125.222 122.428) (width 0.25) (layer "B.Cu") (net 9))
 (segment (start 127.2775 73.3025) (end 130.175 76.2) (width 0.25) (layer "F.Cu") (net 10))
 (segment (start 125.73 73.3025) (end 127.2775 73.3025) (width 0.25) (layer "F.Cu") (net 10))
 (segment (start 137.190479 83.215479) (end 142.397479 83.215479) (width 0.25) (layer "B.Cu") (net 10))
 (segment (start 130.175 76.2) (end 137.190479 83.215479) (width 0.25) (layer "B.Cu") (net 10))
 (segment (start 142.397479 83.215479) (end 144.272 85.09) (width 0.25) (layer "B.Cu") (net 10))
 (segment (start 129.54 73.3025) (end 129.8175 73.3025) (width 0.25) (layer "F.Cu") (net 11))
 (segment (start 129.8175 73.3025) (end 132.715 76.2) (width 0.25) (layer "F.Cu") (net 11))
 (segment (start 132.715 76.2) (end 139.280959 82.765959) (width 0.25) (layer "B.Cu") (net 11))
 (segment (start 145.121981 82.765959) (end 145.871511 83.515489) (width 0.25) (layer "B.Cu") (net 11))
 (segment (start 145.871511 83.515489) (end 145.871511 102.540489) (width 0.25) (layer "B.Cu") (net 11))
 (segment (start 145.871511 102.540489) (end 144.272 104.14) (width 0.25) (layer "B.Cu") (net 11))
 (segment (start 139.280959 82.765959) (end 145.121981 82.765959) (width 0.25) (layer "B.Cu") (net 11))
 (segment (start 133.35 73.3025) (end 133.35 74.295) (width 0.25) (layer "F.Cu") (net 1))
 (segment (start 133.35 74.295) (end 135.255 76.2) (width 0.25) (layer "F.Cu") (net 1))
 (segment (start 146.321031 83.329292) (end 146.321031 121.140969) (width 0.25) (layer "B.Cu") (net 1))
 (segment (start 145.308179 82.316439) (end 146.321031 83.329292) (width 0.25) (layer "B.Cu") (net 1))
 (segment (start 146.321031 121.140969) (end 144.272 123.19) (width 0.25) (layer "B.Cu") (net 1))
 (segment (start 135.255 76.2) (end 141.371439 82.316439) (width 0.25) (layer "B.Cu") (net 1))
 (segment (start 141.371439 82.316439) (end 145.308179 82.316439) (width 0.25) (layer "B.Cu") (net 1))
 (segment (start 137.16 73.3025) (end 137.795 73.9375) (width 0.25) (layer "F.Cu") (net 12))
 (segment (start 137.795 73.9375) (end 137.795 76.2) (width 0.25) (layer "F.Cu") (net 12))
 (segment (start 137.795 76.2) (end 138.919511 77.324511) (width 0.25) (layer "B.Cu") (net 12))
 (segment (start 155.556511 77.324511) (end 163.322 85.09) (width 0.25) (layer "B.Cu") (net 12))
 (segment (start 138.919511 77.324511) (end 155.556511 77.324511) (width 0.25) (layer "B.Cu") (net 12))
 (segment (start 115.13702 69.05952) (end 117.826067 69.05952) (width 0.25) (layer "F.Cu") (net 13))
 (segment (start 131.299511 76.689511) (end 131.934511 77.324511) (width 0.25) (layer "F.Cu") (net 13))
 (segment (start 129.709211 75.075489) (end 130.640789 75.075489) (width 0.25) (layer "F.Cu") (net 13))
 (segment (start 130.640789 75.075489) (end 131.299511 75.734211) (width 0.25) (layer "F.Cu") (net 13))
 (segment (start 131.934511 77.324511) (end 139.210489 77.324511) (width 0.25) (layer "F.Cu") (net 13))
 (segment (start 139.210489 77.324511) (end 140.335 76.2) (width 0.25) (layer "F.Cu") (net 13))
 (segment (start 117.826067 69.05952) (end 121.232027 72.46548) (width 0.25) (layer "F.Cu") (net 13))
 (segment (start 121.232027 72.46548) (end 127.099202 72.46548) (width 0.25) (layer "F.Cu") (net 13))
 (segment (start 114.3 68.2225) (end 115.13702 69.05952) (width 0.25) (layer "F.Cu") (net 13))
 (segment (start 131.299511 75.734211) (end 131.299511 76.689511) (width 0.25) (layer "F.Cu") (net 13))
 (segment (start 127.099202 72.46548) (end 129.709211 75.075489) (width 0.25) (layer "F.Cu") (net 13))
 (segment (start 164.921511 82.371511) (end 164.921511 102.540489) (width 0.25) (layer "B.Cu") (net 13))
 (segment (start 158.75 76.2) (end 164.921511 82.371511) (width 0.25) (layer "B.Cu") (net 13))
 (segment (start 164.921511 102.540489) (end 163.322 104.14) (width 0.25) (layer "B.Cu") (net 13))
 (segment (start 140.335 76.2) (end 158.75 76.2) (width 0.25) (layer "B.Cu") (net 13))
 (segment (start 135.238731 59.385969) (end 138.760969 59.385969) (width 0.25) (layer "F.Cu") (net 14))
 (segment (start 129.5828 68.2225) (end 134.130489 63.674811) (width 0.25) (layer "F.Cu") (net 14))
 (segment (start 138.760969 59.385969) (end 140.335 60.96) (width 0.25) (layer "F.Cu") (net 14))
 (segment (start 134.130489 60.494211) (end 135.238731 59.385969) (width 0.25) (layer "F.Cu") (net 14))
 (segment (start 118.11 68.2225) (end 129.5828 68.2225) (width 0.25) (layer "F.Cu") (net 14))
 (segment (start 134.130489 63.674811) (end 134.130489 60.494211) (width 0.25) (layer "F.Cu") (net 14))
 (segment (start 165.371031 121.140969) (end 163.322 123.19) (width 0.25) (layer "B.Cu") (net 14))
 (segment (start 165.371031 78.572009) (end 165.371031 121.140969) (width 0.25) (layer "B.Cu") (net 14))
 (segment (start 147.759022 60.96) (end 165.371031 78.572009) (width 0.25) (layer "B.Cu") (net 14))
 (segment (start 140.335 60.96) (end 147.759022 60.96) (width 0.25) (layer "B.Cu") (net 14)))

